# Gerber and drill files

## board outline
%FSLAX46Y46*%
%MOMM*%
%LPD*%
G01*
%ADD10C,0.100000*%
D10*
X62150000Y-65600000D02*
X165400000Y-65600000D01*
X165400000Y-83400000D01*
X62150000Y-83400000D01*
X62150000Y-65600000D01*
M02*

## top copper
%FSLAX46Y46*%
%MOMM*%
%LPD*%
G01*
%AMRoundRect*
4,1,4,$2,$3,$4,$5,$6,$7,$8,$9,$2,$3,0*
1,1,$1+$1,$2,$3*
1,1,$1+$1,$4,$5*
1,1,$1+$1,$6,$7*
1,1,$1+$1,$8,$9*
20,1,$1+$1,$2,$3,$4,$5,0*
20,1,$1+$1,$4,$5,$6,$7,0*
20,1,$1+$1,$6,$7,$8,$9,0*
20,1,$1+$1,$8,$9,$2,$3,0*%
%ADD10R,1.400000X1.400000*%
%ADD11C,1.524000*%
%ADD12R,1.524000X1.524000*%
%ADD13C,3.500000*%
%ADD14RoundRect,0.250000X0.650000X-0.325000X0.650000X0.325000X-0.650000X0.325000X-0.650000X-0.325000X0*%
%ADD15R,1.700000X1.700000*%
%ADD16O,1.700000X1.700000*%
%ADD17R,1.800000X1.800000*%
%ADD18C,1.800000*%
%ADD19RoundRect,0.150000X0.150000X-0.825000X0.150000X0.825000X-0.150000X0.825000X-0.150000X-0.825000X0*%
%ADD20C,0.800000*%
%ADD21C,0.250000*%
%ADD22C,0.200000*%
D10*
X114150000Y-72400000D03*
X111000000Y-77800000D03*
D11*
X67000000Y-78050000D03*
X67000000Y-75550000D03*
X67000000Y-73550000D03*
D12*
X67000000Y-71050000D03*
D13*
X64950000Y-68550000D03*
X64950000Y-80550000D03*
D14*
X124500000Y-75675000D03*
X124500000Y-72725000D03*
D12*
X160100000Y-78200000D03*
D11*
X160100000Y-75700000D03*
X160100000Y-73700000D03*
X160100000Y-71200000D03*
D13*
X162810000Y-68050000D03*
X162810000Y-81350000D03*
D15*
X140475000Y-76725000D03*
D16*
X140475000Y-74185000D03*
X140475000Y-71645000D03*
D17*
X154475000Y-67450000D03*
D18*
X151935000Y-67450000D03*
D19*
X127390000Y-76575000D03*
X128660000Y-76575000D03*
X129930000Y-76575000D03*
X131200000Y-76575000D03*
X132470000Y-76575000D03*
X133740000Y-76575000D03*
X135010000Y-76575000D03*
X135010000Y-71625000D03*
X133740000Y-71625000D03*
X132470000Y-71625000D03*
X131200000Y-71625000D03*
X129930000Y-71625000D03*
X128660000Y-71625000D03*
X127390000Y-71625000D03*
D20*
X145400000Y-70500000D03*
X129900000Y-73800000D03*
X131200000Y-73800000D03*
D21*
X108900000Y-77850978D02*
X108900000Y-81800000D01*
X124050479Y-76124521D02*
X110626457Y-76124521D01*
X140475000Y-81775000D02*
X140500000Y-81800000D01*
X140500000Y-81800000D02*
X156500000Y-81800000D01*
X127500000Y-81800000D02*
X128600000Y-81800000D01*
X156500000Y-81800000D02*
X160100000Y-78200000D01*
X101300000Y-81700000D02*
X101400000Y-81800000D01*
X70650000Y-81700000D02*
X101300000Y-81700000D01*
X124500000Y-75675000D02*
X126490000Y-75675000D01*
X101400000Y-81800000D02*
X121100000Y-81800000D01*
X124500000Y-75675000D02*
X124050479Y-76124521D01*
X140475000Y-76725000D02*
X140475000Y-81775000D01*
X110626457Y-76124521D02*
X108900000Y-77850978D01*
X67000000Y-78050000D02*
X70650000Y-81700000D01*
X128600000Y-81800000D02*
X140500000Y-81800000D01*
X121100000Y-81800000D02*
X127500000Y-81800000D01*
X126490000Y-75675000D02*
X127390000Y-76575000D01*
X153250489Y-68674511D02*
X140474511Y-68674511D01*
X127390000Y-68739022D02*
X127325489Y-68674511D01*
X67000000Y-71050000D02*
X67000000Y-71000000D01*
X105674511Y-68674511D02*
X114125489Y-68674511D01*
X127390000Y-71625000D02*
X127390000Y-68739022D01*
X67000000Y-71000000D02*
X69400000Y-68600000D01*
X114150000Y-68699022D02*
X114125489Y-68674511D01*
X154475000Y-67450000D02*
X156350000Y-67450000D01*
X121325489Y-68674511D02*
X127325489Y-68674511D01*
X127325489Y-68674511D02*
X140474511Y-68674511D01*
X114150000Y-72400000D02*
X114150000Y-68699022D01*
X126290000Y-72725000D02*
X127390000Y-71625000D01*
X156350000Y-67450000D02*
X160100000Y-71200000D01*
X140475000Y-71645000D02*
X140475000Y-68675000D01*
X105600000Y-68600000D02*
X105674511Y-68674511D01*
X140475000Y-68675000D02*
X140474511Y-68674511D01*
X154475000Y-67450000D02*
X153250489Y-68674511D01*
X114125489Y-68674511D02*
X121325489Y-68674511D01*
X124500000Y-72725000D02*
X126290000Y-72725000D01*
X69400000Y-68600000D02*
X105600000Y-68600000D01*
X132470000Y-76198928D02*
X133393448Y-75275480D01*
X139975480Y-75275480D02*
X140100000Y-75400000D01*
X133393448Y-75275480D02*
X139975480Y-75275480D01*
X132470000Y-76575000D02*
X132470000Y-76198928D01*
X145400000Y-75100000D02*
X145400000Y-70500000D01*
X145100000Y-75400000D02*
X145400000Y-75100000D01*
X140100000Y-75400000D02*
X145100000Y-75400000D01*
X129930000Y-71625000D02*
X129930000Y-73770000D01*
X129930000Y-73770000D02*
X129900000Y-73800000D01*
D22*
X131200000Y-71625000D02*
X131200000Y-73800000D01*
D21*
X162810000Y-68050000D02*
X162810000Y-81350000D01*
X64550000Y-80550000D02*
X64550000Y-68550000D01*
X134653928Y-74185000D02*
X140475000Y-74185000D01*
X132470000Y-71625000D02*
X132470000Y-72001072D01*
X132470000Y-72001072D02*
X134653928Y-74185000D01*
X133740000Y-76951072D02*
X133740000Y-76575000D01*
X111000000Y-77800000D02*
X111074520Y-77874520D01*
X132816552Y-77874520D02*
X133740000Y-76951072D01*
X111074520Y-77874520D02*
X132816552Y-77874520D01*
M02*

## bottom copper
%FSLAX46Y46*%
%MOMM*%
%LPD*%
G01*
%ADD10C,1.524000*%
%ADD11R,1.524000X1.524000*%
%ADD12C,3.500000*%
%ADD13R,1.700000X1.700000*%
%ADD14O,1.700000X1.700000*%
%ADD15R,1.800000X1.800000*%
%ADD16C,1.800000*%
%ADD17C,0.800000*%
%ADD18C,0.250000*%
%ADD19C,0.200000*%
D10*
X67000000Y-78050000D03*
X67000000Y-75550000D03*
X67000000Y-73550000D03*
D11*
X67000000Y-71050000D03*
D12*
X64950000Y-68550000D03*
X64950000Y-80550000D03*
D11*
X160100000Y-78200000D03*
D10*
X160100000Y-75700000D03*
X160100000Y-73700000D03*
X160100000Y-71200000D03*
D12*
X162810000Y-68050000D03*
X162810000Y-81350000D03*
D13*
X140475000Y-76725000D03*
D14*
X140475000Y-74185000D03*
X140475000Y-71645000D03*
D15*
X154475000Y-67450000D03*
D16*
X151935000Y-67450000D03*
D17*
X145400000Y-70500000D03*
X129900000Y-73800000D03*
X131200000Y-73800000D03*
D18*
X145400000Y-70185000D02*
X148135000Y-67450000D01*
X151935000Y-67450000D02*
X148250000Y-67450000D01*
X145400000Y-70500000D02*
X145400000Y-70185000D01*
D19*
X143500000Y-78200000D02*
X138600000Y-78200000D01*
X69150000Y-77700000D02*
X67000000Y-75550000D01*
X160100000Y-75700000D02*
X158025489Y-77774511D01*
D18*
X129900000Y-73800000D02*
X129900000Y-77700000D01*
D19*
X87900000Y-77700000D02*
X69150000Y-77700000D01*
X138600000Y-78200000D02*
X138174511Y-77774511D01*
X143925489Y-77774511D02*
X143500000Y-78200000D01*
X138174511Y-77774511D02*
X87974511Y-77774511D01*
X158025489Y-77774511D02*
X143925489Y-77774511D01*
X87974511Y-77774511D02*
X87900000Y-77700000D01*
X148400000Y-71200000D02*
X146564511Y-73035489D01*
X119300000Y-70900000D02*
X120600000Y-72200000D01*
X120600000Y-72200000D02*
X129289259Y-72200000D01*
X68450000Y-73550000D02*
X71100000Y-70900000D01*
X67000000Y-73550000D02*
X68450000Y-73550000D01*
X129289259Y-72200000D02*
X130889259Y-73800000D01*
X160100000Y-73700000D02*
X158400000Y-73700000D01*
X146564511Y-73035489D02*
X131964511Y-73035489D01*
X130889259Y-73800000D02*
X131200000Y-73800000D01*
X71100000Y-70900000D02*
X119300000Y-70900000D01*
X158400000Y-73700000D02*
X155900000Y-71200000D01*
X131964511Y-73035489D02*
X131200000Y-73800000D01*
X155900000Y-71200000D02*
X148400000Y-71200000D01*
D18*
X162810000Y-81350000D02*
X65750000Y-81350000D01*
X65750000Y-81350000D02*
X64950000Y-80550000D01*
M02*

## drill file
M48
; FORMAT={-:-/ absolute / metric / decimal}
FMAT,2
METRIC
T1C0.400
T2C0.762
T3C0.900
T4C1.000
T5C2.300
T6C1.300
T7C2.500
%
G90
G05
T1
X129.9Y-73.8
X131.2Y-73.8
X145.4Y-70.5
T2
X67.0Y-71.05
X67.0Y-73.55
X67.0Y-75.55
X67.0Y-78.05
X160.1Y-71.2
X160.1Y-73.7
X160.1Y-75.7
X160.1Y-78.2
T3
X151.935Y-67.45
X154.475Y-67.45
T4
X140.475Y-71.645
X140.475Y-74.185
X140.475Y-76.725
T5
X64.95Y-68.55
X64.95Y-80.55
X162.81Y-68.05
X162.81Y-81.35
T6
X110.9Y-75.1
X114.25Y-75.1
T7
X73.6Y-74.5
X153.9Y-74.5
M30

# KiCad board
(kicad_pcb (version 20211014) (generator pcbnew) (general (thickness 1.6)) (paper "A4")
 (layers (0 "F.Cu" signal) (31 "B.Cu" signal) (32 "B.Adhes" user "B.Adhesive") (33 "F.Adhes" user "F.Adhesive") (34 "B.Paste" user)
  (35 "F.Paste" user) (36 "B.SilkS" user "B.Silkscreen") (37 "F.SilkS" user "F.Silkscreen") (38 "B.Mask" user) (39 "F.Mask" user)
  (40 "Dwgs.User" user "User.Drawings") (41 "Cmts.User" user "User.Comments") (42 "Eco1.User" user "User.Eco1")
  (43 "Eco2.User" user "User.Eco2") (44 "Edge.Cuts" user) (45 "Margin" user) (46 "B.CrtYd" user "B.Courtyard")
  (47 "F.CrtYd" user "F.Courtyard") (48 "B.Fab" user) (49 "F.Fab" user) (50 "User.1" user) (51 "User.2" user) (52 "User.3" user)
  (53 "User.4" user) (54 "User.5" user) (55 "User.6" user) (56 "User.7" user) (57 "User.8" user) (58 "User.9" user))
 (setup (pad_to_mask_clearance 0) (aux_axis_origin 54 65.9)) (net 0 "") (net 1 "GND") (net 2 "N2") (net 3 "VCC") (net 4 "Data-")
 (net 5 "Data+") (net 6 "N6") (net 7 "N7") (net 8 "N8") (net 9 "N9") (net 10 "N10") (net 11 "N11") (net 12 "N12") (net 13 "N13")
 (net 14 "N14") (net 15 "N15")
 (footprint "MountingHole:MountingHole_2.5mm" (layer "F.Cu") (at 153.9 74.5)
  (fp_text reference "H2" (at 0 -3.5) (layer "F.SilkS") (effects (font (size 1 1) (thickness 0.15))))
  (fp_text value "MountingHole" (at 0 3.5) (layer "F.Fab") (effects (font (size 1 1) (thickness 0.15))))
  (pad "" np_thru_hole circle (at 0 0) (size 2.5 2.5) (drill 2.5) (layers *.Cu *.Mask)))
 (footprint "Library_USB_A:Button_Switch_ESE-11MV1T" (layer "F.Cu") (at 112.7 75.1 180)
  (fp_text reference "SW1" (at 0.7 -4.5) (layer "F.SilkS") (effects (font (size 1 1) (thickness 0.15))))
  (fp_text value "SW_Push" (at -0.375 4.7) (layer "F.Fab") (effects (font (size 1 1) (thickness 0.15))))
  (pad "" np_thru_hole circle (at -1.55 0 90) (size 1.3 1.3) (drill 1.3) (layers F&B.Cu *.Mask))
  (pad "" np_thru_hole circle (at 1.8 0 90) (size 1.3 1.3) (drill 1.3) (layers F&B.Cu *.Mask))
  (pad "1" smd rect (at -1.45 2.7 90) (size 1.4 1.4) (layers "F.Cu" "F.Paste" "F.Mask") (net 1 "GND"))
  (pad "2" smd rect (at 1.7 -2.7 90) (size 1.4 1.4) (layers "F.Cu" "F.Paste" "F.Mask") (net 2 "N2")))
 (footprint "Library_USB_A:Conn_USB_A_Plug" (layer "F.Cu") (at 67.05 74.55 -90)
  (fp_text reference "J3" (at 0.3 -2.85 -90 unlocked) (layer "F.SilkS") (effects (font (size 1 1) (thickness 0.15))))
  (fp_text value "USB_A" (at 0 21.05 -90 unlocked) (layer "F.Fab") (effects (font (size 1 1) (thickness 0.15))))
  (pad "1" thru_hole circle (at 3.5 0.05 270) (size 1.524 1.524) (drill 0.762) (layers *.Cu *.Mask) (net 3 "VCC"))
  (pad "2" thru_hole circle (at 1 0.05 270) (size 1.524 1.524) (drill 0.762) (layers *.Cu *.Mask) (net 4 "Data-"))
  (pad "3" thru_hole circle (at -1 0.05 270) (size 1.524 1.524) (drill 0.762) (layers *.Cu *.Mask) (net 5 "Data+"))
  (pad "4" thru_hole rect (at -3.5 0.05 270) (size 1.524 1.524) (drill 0.762) (layers *.Cu *.Mask) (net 1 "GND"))
  (pad "5" thru_hole circle (at -6 2.1 270) (size 3.5 3.5) (drill 2.3) (layers *.Cu *.Mask) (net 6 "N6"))
  (pad "5" thru_hole circle (at 6 2.1 270) (size 3.5 3.5) (drill 2.3) (layers *.Cu *.Mask) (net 6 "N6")))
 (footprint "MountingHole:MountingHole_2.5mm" (layer "F.Cu") (at 73.6 74.5)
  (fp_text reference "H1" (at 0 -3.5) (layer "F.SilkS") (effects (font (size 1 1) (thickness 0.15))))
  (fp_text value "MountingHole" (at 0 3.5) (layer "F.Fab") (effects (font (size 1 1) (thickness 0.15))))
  (pad "" np_thru_hole circle (at 0 0) (size 2.5 2.5) (drill 2.5) (layers *.Cu *.Mask)))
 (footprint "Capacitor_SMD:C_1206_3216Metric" (layer "F.Cu") (at 124.5 74.2 90)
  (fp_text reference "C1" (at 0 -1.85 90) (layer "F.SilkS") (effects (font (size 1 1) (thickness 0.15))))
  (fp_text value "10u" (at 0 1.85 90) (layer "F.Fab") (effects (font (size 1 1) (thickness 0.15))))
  (pad "1" smd roundrect (at -1.475 0 90) (size 1.15 1.8) (layers "F.Cu" "F.Paste" "F.Mask") (roundrect_rratio 0.2173913043) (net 3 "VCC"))
  (pad "2" smd roundrect (at 1.475 0 90) (size 1.15 1.8) (layers "F.Cu" "F.Paste" "F.Mask") (roundrect_rratio 0.2173913043) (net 1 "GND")))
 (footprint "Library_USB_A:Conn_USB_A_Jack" (layer "F.Cu") (at 160.1 74.7 90)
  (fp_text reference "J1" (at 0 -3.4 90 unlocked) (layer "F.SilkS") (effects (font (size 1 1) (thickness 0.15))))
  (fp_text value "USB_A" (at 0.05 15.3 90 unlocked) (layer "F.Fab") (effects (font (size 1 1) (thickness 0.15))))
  (pad "1" thru_hole rect (at -3.5 0 90) (size 1.524 1.524) (drill 0.762) (layers *.Cu *.Mask) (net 3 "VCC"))
  (pad "2" thru_hole circle (at -1 0 90) (size 1.524 1.524) (drill 0.762) (layers *.Cu *.Mask) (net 4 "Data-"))
  (pad "3" thru_hole circle (at 1 0 90) (size 1.524 1.524) (drill 0.762) (layers *.Cu *.Mask) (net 5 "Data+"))
  (pad "4" thru_hole circle (at 3.5 0 90) (size 1.524 1.524) (drill 0.762) (layers *.Cu *.Mask) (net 1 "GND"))
  (pad "5" thru_hole circle (at 6.65 2.71 90) (size 3.5 3.5) (drill 2.3) (layers *.Cu *.Mask) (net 6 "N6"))
  (pad "5" thru_hole circle (at -6.65 2.71 90) (size 3.5 3.5) (drill 2.3) (layers *.Cu *.Mask) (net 6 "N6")))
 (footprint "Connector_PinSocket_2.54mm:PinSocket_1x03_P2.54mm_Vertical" (layer "F.Cu") (at 140.475 76.725 180)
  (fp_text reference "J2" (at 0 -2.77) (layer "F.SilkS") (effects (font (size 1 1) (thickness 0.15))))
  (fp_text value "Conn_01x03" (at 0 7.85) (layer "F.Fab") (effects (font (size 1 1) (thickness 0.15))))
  (pad "1" thru_hole rect (at 0 0 180) (size 1.7 1.7) (drill 1) (layers *.Cu *.Mask) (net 3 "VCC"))
  (pad "2" thru_hole oval (at 0 2.54 180) (size 1.7 1.7) (drill 1) (layers *.Cu *.Mask) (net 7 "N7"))
  (pad "3" thru_hole oval (at 0 5.08 180) (size 1.7 1.7) (drill 1) (layers *.Cu *.Mask) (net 1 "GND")))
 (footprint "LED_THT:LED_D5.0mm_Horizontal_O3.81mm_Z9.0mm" (layer "F.Cu") (at 154.475 67.45 180)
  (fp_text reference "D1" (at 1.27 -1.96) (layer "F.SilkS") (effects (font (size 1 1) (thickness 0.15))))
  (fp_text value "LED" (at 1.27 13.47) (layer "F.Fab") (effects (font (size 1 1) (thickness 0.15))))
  (pad "1" thru_hole rect (at 0 0 180) (size 1.8 1.8) (drill 0.9) (layers *.Cu *.Mask) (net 1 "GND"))
  (pad "2" thru_hole circle (at 2.54 0 180) (size 1.8 1.8) (drill 0.9) (layers *.Cu *.Mask) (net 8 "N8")))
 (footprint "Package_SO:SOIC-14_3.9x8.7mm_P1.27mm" (layer "F.Cu") (at 131.2 74.1 90)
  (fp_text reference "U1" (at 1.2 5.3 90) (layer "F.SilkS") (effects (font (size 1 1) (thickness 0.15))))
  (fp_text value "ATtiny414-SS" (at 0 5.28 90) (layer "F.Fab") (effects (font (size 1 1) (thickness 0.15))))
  (pad "1" smd roundrect (at -2.475 -3.81 90) (size 1.95 0.6) (layers "F.Cu" "F.Paste" "F.Mask") (roundrect_rratio 0.25) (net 3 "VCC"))
  (pad "2" smd roundrect (at -2.475 -2.54 90) (size 1.95 0.6) (layers "F.Cu" "F.Paste" "F.Mask") (roundrect_rratio 0.25) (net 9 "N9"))
  (pad "3" smd roundrect (at -2.475 -1.27 90) (size 1.95 0.6) (layers "F.Cu" "F.Paste" "F.Mask") (roundrect_rratio 0.25) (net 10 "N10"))
  (pad "4" smd roundrect (at -2.475 0 90) (size 1.95 0.6) (layers "F.Cu" "F.Paste" "F.Mask") (roundrect_rratio 0.25) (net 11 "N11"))
  (pad "5" smd roundrect (at -2.475 1.27 90) (size 1.95 0.6) (layers "F.Cu" "F.Paste" "F.Mask") (roundrect_rratio 0.25) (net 8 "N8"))
  (pad "6" smd roundrect (at -2.475 2.54 90) (size 1.95 0.6) (layers "F.Cu" "F.Paste" "F.Mask") (roundrect_rratio 0.25) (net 2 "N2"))
  (pad "7" smd roundrect (at -2.475 3.81 90) (size 1.95 0.6) (layers "F.Cu" "F.Paste" "F.Mask") (roundrect_rratio 0.25) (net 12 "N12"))
  (pad "8" smd roundrect (at 2.475 3.81 90) (size 1.95 0.6) (layers "F.Cu" "F.Paste" "F.Mask") (roundrect_rratio 0.25) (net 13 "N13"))
  (pad "9" smd roundrect (at 2.475 2.54 90) (size 1.95 0.6) (layers "F.Cu" "F.Paste" "F.Mask") (roundrect_rratio 0.25) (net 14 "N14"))
  (pad "10" smd roundrect (at 2.475 1.27 90) (size 1.95 0.6) (layers "F.Cu" "F.Paste" "F.Mask") (roundrect_rratio 0.25) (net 7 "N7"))
  (pad "11" smd roundrect (at 2.475 0 90) (size 1.95 0.6) (layers "F.Cu" "F.Paste" "F.Mask") (roundrect_rratio 0.25) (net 5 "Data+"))
  (pad "12" smd roundrect (at 2.475 -1.27 90) (size 1.95 0.6) (layers "F.Cu" "F.Paste" "F.Mask") (roundrect_rratio 0.25) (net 4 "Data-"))
  (pad "13" smd roundrect (at 2.475 -2.54 90) (size 1.95 0.6) (layers "F.Cu" "F.Paste" "F.Mask") (roundrect_rratio 0.25) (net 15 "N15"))
  (pad "14" smd roundrect (at 2.475 -3.81 90) (size 1.95 0.6) (layers "F.Cu" "F.Paste" "F.Mask") (roundrect_rratio 0.25) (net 1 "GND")))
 (gr_rect (start 62.15 65.6) (end 165.4 83.4) (layer "Edge.Cuts") (width 0.1) (fill none))
 (segment (start 108.9 77.850978) (end 108.9 81.8) (width 0.25) (layer "F.Cu") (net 3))
 (segment (start 124.050479 76.124521) (end 110.626457 76.124521) (width 0.25) (layer "F.Cu") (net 3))
 (segment (start 140.475 81.775) (end 140.5 81.8) (width 0.25) (layer "F.Cu") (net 3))
 (segment (start 140.5 81.8) (end 156.5 81.8) (width 0.25) (layer "F.Cu") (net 3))
 (segment (start 127.5 81.8) (end 128.6 81.8) (width 0.25) (layer "F.Cu") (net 3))
 (segment (start 156.5 81.8) (end 160.1 78.2) (width 0.25) (layer "F.Cu") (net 3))
 (segment (start 101.3 81.7) (end 101.4 81.8) (width 0.25) (layer "F.Cu") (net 3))
 (segment (start 70.65 81.7) (end 101.3 81.7) (width 0.25) (layer "F.Cu") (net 3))
 (segment (start 124.5 75.675) (end 126.49 75.675) (width 0.25) (layer "F.Cu") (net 3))
 (segment (start 101.4 81.8) (end 121.1 81.8) (width 0.25) (layer "F.Cu") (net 3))
 (segment (start 124.5 75.675) (end 124.050479 76.124521) (width 0.25) (layer "F.Cu") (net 3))
 (segment (start 140.475 76.725) (end 140.475 81.775) (width 0.25) (layer "F.Cu") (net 3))
 (segment (start 110.626457 76.124521) (end 108.9 77.850978) (width 0.25) (layer "F.Cu") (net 3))
 (segment (start 67 78.05) (end 70.65 81.7) (width 0.25) (layer "F.Cu") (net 3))
 (segment (start 128.6 81.8) (end 140.5 81.8) (width 0.25) (layer "F.Cu") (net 3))
 (segment (start 121.1 81.8) (end 127.5 81.8) (width 0.25) (layer "F.Cu") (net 3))
 (segment (start 126.49 75.675) (end 127.39 76.575) (width 0.25) (layer "F.Cu") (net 3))
 (segment (start 153.250489 68.674511) (end 140.474511 68.674511) (width 0.25) (layer "F.Cu") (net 1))
 (segment (start 127.39 68.739022) (end 127.325489 68.674511) (width 0.25) (layer "F.Cu") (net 1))
 (segment (start 67 71.05) (end 67 71) (width 0.25) (layer "F.Cu") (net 1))
 (segment (start 105.674511 68.674511) (end 114.125489 68.674511) (width 0.25) (layer "F.Cu") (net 1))
 (segment (start 127.39 71.625) (end 127.39 68.739022) (width 0.25) (layer "F.Cu") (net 1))
 (segment (start 67 71) (end 69.4 68.6) (width 0.25) (layer "F.Cu") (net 1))
 (segment (start 114.15 68.699022) (end 114.125489 68.674511) (width 0.25) (layer "F.Cu") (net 1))
 (segment (start 154.475 67.45) (end 156.35 67.45) (width 0.25) (layer "F.Cu") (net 1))
 (segment (start 121.325489 68.674511) (end 127.325489 68.674511) (width 0.25) (layer "F.Cu") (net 1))
 (segment (start 127.325489 68.674511) (end 140.474511 68.674511) (width 0.25) (layer "F.Cu") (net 1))
 (segment (start 114.15 72.4) (end 114.15 68.699022) (width 0.25) (layer "F.Cu") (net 1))
 (segment (start 126.29 72.725) (end 127.39 71.625) (width 0.25) (layer "F.Cu") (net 1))
 (segment (start 156.35 67.45) (end 160.1 71.2) (width 0.25) (layer "F.Cu") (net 1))
 (segment (start 140.475 71.645) (end 140.475 68.675) (width 0.25) (layer "F.Cu") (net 1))
 (segment (start 105.6 68.6) (end 105.674511 68.674511) (width 0.25) (layer "F.Cu") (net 1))
 (segment (start 140.475 68.675) (end 140.474511 68.674511) (width 0.25) (layer "F.Cu") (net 1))
 (segment (start 154.475 67.45) (end 153.250489 68.674511) (width 0.25) (layer "F.Cu") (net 1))
 (segment (start 114.125489 68.674511) (end 121.325489 68.674511) (width 0.25) (layer "F.Cu") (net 1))
 (segment (start 124.5 72.725) (end 126.29 72.725) (width 0.25) (layer "F.Cu") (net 1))
 (segment (start 69.4 68.6) (end 105.6 68.6) (width 0.25) (layer "F.Cu") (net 1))
 (segment (start 132.47 76.198928) (end 133.393448 75.27548) (width 0.25) (layer "F.Cu") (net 8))
 (segment (start 139.97548 75.27548) (end 140.1 75.4) (width 0.25) (layer "F.Cu") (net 8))
 (segment (start 133.393448 75.27548) (end 139.97548 75.27548) (width 0.25) (layer "F.Cu") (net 8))
 (segment (start 132.47 76.575) (end 132.47 76.198928) (width 0.25) (layer "F.Cu") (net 8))
 (segment (start 145.4 75.1) (end 145.4 70.5) (width 0.25) (layer "F.Cu") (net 8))
 (segment (start 145.1 75.4) (end 145.4 75.1) (width 0.25) (layer "F.Cu") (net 8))
 (segment (start 140.1 75.4) (end 145.1 75.4) (width 0.25) (layer "F.Cu") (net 8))
 (via (at 145.4 70.5) (size 0.8) (drill 0.4) (layers "F.Cu" "B.Cu") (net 8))
 (segment (start 145.4 70.185) (end 148.135 67.45) (width 0.25) (layer "B.Cu") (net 8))
 (segment (start 151.935 67.45) (end 148.25 67.45) (width 0.25) (layer "B.Cu") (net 8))
 (segment (start 145.4 70.5) (end 145.4 70.185) (width 0.25) (layer "B.Cu") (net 8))
 (segment (start 129.93 71.625) (end 129.93 73.77) (width 0.25) (layer "F.Cu") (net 4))
 (segment (start 129.93 73.77) (end 129.9 73.8) (width 0.25) (layer "F.Cu") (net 4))
 (via (at 129.9 73.8) (size 0.8) (drill 0.4) (layers "F.Cu" "B.Cu") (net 4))
 (segment (start 143.5 78.2) (end 138.6 78.2) (width 0.2) (layer "B.Cu") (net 4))
 (segment (start 69.15 77.7) (end 67 75.55) (width 0.2) (layer "B.Cu") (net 4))
 (segment (start 160.1 75.7) (end 158.025489 77.774511) (width 0.2) (layer "B.Cu") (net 4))
 (segment (start 129.9 73.8) (end 129.9 77.7) (width 0.25) (layer "B.Cu") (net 4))
 (segment (start 87.9 77.7) (end 69.15 77.7) (width 0.2) (layer "B.Cu") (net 4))
 (segment (start 138.6 78.2) (end 138.174511 77.774511) (width 0.2) (layer "B.Cu") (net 4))
 (segment (start 143.925489 77.774511) (end 143.5 78.2) (width 0.2) (layer "B.Cu") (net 4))
 (segment (start 138.174511 77.774511) (end 87.974511 77.774511) (width 0.2) (layer "B.Cu") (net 4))
 (segment (start 158.025489 77.774511) (end 143.925489 77.774511) (width 0.2) (layer "B.Cu") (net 4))
 (segment (start 87.974511 77.774511) (end 87.9 77.7) (width 0.2) (layer "B.Cu") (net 4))
 (segment (start 131.2 71.625) (end 131.2 73.8) (width 0.2) (layer "F.Cu") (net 5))
 (via (at 131.2 73.8) (size 0.8) (drill 0.4) (layers "F.Cu" "B.Cu") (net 5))
 (segment (start 148.4 71.2) (end 146.564511 73.035489) (width 0.2) (layer "B.Cu") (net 5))
 (segment (start 119.3 70.9) (end 120.6 72.2) (width 0.2) (layer "B.Cu") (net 5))
 (segment (start 120.6 72.2) (end 129.289259 72.2) (width 0.2) (layer "B.Cu") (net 5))
 (segment (start 68.45 73.55) (end 71.1 70.9) (width 0.2) (layer "B.Cu") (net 5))
 (segment (start 67 73.55) (end 68.45 73.55) (width 0.2) (layer "B.Cu") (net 5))
 (segment (start 129.289259 72.2) (end 130.889259 73.8) (width 0.2) (layer "B.Cu") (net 5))
 (segment (start 160.1 73.7) (end 158.4 73.7) (width 0.2) (layer "B.Cu") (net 5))
 (segment (start 146.564511 73.035489) (end 131.964511 73.035489) (width 0.2) (layer "B.Cu") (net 5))
 (segment (start 130.889259 73.8) (end 131.2 73.8) (width 0.2) (layer "B.Cu") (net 5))
 (segment (start 71.1 70.9) (end 119.3 70.9) (width 0.2) (layer "B.Cu") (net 5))
 (segment (start 158.4 73.7) (end 155.9 71.2) (width 0.2) (layer "B.Cu") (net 5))
 (segment (start 131.964511 73.035489) (end 131.2 73.8) (width 0.2) (layer "B.Cu") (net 5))
 (segment (start 155.9 71.2) (end 148.4 71.2) (width 0.2) (layer "B.Cu") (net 5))
 (segment (start 162.81 68.05) (end 162.81 81.35) (width 0.25) (layer "F.Cu") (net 6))
 (segment (start 64.55 80.55) (end 64.55 68.55) (width 0.25) (layer "F.Cu") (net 6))
 (segment (start 162.81 81.35) (end 65.75 81.35) (width 0.25) (layer "B.Cu") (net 6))
 (segment (start 65.75 81.35) (end 64.95 80.55) (width 0.25) (layer "B.Cu") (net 6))
 (segment (start 134.653928 74.185) (end 140.475 74.185) (width 0.25) (layer "F.Cu") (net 7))
 (segment (start 132.47 71.625) (end 132.47 72.001072) (width 0.25) (layer "F.Cu") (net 7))
 (segment (start 132.47 72.001072) (end 134.653928 74.185) (width 0.25) (layer "F.Cu") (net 7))
 (segment (start 133.74 76.951072) (end 133.74 76.575) (width 0.25) (layer "F.Cu") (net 2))
 (segment (start 111 77.8) (end 111.07452 77.87452) (width 0.25) (layer "F.Cu") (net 2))
 (segment (start 132.816552 77.87452) (end 133.74 76.951072) (width 0.25) (layer "F.Cu") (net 2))
 (segment (start 111.07452 77.87452) (end 132.816552 77.87452) (width 0.25) (layer "F.Cu") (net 2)))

